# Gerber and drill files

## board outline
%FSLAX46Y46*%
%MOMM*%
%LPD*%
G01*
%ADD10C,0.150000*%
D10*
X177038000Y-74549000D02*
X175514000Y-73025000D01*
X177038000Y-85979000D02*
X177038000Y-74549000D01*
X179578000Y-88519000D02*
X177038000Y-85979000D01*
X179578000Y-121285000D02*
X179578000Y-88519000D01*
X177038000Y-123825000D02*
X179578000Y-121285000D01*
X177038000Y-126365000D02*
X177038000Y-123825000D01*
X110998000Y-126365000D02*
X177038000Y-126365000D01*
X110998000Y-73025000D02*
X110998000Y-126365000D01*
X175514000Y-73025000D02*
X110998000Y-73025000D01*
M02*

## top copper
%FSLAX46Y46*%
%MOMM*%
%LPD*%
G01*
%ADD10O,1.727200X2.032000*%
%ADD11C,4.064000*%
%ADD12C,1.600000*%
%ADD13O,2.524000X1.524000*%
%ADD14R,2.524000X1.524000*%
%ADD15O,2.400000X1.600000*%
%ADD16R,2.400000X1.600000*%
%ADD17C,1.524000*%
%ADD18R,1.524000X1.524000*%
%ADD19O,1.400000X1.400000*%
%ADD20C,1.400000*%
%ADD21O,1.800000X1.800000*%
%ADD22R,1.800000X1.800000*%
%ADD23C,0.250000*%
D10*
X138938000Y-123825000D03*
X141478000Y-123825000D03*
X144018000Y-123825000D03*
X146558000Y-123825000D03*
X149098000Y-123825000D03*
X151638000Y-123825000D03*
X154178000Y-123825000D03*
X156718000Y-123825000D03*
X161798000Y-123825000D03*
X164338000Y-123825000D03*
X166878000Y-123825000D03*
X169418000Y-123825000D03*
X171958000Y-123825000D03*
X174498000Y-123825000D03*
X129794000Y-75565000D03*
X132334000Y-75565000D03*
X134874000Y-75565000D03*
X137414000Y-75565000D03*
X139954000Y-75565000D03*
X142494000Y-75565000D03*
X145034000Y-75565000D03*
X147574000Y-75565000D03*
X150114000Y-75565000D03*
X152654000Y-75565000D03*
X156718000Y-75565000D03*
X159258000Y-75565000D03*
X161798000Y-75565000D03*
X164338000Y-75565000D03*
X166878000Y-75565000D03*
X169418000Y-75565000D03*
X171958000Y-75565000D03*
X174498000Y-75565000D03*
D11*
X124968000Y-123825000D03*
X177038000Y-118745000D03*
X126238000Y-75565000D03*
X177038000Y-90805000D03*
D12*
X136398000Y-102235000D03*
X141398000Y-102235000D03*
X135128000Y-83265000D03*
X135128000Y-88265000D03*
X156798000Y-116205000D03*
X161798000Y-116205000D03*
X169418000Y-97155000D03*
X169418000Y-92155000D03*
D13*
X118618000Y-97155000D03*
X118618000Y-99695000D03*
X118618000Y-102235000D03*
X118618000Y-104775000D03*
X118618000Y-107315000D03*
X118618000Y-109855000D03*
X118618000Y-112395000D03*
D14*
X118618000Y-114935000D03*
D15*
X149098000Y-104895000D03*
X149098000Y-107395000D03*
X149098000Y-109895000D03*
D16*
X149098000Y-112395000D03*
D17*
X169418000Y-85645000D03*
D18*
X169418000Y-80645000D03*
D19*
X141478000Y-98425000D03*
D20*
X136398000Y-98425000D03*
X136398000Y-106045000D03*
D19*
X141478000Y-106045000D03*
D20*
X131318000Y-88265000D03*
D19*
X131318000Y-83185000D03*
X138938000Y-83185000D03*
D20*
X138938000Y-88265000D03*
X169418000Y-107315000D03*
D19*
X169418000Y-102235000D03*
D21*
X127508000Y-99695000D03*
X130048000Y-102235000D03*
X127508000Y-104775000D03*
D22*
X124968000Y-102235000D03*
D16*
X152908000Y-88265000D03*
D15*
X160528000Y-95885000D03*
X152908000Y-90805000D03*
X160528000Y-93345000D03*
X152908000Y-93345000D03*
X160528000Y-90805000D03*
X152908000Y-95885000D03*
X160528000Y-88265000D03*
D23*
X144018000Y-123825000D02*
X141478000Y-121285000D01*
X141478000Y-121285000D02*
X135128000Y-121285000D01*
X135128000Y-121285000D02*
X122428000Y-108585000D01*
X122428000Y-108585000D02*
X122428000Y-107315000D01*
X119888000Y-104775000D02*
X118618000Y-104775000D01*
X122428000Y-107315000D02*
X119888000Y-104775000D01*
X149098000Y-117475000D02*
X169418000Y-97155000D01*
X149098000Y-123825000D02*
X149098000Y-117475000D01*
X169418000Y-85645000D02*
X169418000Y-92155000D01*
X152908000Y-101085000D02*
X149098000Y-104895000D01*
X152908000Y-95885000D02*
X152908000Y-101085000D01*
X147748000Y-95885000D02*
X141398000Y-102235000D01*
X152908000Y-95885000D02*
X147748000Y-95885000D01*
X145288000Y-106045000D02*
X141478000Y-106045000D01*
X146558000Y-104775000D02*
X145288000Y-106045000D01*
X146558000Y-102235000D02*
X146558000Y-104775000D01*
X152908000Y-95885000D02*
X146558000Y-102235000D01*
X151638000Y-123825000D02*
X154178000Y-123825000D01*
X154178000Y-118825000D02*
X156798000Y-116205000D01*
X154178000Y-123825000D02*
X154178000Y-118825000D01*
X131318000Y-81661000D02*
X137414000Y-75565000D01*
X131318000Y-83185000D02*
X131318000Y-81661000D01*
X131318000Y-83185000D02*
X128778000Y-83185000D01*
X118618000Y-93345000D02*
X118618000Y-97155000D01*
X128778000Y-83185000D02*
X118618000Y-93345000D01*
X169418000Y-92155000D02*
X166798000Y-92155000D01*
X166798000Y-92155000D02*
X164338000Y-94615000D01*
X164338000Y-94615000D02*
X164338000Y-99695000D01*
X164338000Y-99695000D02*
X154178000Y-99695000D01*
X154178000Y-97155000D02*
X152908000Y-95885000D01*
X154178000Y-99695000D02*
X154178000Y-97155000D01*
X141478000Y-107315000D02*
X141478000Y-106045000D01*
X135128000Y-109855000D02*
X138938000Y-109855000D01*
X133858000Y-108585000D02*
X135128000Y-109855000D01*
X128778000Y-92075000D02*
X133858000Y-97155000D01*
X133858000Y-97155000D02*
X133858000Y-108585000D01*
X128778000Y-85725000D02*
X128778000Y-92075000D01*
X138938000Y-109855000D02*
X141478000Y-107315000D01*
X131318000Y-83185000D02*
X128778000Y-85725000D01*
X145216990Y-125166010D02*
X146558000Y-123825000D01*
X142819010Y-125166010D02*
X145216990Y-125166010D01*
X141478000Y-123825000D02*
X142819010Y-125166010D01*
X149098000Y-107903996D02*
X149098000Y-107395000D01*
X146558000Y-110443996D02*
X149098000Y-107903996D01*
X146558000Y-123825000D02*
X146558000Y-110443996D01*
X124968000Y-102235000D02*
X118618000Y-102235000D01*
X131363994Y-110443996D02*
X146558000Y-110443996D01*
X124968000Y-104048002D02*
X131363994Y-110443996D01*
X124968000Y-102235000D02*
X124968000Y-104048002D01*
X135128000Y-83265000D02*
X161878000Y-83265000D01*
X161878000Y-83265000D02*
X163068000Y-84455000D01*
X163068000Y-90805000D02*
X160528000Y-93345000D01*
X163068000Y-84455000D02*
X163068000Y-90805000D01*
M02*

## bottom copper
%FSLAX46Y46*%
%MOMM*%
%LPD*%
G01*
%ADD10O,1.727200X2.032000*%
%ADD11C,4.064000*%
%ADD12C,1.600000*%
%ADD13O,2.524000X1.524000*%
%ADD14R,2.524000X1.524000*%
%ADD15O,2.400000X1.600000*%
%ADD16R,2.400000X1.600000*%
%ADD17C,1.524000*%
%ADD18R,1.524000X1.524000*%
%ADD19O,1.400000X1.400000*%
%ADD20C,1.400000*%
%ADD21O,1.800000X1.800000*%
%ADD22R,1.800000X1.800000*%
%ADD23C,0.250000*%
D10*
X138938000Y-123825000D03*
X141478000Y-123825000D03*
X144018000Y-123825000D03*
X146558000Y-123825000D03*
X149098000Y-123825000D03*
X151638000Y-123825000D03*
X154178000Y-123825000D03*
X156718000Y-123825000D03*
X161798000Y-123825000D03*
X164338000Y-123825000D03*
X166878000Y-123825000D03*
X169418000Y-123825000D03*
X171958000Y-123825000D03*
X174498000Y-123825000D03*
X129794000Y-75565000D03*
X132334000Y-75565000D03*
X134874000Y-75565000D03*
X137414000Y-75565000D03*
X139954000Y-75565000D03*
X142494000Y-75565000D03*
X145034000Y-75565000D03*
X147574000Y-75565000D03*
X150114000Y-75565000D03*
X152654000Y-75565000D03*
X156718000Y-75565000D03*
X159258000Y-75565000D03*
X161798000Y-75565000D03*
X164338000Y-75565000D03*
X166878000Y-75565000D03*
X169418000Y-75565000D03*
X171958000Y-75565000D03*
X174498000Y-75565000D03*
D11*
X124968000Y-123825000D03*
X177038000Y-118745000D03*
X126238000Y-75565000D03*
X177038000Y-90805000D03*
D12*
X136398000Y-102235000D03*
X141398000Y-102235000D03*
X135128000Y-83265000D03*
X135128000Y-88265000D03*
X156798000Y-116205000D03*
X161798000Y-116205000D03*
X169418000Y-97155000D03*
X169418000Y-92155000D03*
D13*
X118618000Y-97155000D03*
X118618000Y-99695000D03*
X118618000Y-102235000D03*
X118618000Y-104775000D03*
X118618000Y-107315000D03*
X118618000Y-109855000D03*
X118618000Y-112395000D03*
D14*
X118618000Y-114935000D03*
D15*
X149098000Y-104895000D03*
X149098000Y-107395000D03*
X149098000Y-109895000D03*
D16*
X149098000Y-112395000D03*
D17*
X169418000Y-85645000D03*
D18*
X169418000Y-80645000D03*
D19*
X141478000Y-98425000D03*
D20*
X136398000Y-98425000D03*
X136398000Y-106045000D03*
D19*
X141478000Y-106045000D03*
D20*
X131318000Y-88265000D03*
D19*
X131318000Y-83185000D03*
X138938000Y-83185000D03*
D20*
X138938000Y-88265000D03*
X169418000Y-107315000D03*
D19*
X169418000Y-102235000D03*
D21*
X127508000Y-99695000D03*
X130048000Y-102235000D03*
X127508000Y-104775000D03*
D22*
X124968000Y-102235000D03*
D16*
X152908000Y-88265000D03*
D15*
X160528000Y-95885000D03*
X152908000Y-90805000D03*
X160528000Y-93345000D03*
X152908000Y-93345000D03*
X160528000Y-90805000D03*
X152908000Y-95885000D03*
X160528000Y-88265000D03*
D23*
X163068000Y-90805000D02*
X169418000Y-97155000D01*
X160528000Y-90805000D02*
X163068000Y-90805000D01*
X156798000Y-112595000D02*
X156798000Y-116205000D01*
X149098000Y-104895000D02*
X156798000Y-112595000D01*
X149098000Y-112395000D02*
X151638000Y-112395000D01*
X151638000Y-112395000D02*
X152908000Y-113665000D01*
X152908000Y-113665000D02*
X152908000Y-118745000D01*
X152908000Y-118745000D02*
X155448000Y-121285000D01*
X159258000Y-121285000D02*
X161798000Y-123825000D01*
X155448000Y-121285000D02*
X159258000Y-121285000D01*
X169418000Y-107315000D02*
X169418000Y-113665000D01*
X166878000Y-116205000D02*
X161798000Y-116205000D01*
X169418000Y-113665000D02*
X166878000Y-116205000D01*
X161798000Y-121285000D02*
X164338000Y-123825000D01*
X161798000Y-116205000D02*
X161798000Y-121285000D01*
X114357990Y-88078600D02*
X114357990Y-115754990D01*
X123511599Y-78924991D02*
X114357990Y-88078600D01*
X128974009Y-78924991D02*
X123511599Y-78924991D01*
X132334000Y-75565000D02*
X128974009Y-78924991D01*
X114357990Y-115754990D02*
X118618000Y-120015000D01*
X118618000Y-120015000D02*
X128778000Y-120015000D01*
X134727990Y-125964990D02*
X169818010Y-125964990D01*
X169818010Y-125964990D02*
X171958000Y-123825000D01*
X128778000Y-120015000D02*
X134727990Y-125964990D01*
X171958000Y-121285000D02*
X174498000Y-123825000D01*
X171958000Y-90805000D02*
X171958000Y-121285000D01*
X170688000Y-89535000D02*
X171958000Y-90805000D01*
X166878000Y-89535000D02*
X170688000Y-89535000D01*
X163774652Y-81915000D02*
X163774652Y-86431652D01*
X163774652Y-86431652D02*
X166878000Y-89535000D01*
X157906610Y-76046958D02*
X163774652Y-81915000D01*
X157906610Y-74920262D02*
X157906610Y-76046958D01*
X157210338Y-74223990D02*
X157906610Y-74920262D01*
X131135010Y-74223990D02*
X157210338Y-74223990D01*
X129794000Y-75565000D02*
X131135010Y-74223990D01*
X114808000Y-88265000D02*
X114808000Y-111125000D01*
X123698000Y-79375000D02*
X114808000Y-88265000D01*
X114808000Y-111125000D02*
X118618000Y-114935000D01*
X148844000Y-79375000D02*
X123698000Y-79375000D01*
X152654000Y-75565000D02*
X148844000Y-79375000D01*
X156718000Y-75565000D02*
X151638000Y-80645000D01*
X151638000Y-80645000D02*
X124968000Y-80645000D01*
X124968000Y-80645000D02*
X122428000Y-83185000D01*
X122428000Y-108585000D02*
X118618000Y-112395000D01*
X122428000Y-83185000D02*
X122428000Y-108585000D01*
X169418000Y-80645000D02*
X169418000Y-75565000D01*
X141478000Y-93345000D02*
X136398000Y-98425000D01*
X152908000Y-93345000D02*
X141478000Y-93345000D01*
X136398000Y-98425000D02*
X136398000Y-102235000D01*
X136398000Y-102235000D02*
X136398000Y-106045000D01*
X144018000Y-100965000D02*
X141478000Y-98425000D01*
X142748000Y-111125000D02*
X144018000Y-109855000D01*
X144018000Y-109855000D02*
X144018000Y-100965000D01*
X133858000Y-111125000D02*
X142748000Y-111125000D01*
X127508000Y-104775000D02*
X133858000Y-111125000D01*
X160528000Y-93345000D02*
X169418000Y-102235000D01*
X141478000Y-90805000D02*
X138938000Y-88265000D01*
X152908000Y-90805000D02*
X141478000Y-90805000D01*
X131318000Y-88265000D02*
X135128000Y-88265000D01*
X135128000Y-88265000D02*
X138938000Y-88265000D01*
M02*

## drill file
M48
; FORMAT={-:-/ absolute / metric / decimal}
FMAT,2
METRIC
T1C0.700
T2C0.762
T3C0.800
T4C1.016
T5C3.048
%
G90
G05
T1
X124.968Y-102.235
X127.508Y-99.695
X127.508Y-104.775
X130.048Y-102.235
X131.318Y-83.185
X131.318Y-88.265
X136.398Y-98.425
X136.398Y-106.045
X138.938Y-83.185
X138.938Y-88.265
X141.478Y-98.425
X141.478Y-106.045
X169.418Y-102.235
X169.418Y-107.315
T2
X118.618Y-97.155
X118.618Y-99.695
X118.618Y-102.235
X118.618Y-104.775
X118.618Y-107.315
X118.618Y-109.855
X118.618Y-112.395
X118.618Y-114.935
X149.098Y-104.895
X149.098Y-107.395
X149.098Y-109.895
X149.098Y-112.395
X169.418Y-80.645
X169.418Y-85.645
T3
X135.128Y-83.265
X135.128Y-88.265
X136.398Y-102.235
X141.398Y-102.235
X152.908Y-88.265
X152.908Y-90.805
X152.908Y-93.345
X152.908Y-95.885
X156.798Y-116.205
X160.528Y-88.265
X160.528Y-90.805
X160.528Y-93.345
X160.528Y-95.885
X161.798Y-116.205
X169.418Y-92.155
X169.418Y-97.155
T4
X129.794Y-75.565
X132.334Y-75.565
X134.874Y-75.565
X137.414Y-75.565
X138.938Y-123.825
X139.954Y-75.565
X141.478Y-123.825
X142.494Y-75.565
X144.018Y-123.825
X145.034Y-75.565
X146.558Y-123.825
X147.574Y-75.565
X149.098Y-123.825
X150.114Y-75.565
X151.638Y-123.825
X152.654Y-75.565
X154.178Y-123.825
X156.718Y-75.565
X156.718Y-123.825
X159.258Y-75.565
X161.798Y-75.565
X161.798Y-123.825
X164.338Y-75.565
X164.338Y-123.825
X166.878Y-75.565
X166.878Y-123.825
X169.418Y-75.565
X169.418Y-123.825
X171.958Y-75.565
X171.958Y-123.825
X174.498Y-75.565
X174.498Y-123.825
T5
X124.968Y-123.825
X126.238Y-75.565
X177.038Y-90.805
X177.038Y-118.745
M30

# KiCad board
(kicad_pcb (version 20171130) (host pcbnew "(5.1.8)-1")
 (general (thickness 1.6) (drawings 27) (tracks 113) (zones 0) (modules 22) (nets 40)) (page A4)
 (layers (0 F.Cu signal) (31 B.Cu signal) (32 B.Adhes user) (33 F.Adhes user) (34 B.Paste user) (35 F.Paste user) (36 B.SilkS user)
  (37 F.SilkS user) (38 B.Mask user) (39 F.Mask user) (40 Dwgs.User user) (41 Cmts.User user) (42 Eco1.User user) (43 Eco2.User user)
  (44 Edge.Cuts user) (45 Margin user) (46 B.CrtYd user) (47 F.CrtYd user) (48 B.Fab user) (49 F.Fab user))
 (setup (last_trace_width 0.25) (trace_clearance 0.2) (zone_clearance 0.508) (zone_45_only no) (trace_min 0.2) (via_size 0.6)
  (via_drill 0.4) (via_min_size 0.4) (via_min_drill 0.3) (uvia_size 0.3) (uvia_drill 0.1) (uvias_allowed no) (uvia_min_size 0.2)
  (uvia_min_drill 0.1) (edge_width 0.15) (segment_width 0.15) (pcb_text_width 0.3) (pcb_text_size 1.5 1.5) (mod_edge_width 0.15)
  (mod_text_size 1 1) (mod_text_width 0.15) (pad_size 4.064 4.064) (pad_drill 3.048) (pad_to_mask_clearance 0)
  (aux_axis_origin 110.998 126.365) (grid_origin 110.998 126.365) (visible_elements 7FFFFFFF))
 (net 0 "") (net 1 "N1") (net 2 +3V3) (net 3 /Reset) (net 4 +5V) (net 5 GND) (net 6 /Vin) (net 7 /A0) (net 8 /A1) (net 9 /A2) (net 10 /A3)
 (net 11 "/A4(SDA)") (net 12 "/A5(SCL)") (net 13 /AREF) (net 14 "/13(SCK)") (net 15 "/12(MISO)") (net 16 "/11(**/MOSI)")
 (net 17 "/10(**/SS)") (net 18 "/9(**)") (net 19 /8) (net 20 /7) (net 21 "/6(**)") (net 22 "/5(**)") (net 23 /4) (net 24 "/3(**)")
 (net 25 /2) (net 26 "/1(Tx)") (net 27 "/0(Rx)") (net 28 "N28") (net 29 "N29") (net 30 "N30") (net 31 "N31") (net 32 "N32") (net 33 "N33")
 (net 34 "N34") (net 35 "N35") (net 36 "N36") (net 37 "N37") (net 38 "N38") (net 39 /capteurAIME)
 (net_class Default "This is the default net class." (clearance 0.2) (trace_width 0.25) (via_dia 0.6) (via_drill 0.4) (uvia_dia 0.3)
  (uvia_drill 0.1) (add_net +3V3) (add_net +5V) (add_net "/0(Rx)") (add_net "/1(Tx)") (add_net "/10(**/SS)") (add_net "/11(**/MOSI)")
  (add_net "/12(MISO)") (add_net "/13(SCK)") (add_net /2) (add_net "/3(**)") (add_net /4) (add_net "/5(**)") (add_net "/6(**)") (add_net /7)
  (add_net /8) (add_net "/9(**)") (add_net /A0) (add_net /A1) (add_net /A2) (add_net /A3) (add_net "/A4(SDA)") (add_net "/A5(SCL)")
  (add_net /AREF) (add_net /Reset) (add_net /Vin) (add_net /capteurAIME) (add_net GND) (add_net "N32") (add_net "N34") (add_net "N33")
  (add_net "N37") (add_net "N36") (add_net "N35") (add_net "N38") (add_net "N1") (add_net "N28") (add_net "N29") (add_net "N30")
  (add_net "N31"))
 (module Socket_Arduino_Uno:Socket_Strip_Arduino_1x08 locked (layer F.Cu) (at 138.938 123.825)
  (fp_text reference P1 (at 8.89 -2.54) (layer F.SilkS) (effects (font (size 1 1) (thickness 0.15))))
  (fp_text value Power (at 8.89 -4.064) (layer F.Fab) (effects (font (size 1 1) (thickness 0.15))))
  (pad 1 thru_hole oval (at 0 0) (size 1.7272 2.032) (drill 1.016) (layers *.Cu *.Mask F.SilkS) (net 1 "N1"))
  (pad 2 thru_hole oval (at 2.54 0) (size 1.7272 2.032) (drill 1.016) (layers *.Cu *.Mask F.SilkS) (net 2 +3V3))
  (pad 3 thru_hole oval (at 5.08 0) (size 1.7272 2.032) (drill 1.016) (layers *.Cu *.Mask F.SilkS) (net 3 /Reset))
  (pad 4 thru_hole oval (at 7.62 0) (size 1.7272 2.032) (drill 1.016) (layers *.Cu *.Mask F.SilkS) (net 2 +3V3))
  (pad 5 thru_hole oval (at 10.16 0) (size 1.7272 2.032) (drill 1.016) (layers *.Cu *.Mask F.SilkS) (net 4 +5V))
  (pad 6 thru_hole oval (at 12.7 0) (size 1.7272 2.032) (drill 1.016) (layers *.Cu *.Mask F.SilkS) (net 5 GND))
  (pad 7 thru_hole oval (at 15.24 0) (size 1.7272 2.032) (drill 1.016) (layers *.Cu *.Mask F.SilkS) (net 5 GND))
  (pad 8 thru_hole oval (at 17.78 0) (size 1.7272 2.032) (drill 1.016) (layers *.Cu *.Mask F.SilkS) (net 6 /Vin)))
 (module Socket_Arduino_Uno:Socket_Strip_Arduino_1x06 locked (layer F.Cu) (at 161.798 123.825)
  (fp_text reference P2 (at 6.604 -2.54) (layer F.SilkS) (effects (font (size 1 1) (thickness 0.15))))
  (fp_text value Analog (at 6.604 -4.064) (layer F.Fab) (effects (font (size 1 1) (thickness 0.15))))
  (pad 1 thru_hole oval (at 0 0) (size 1.7272 2.032) (drill 1.016) (layers *.Cu *.Mask F.SilkS) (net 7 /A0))
  (pad 2 thru_hole oval (at 2.54 0) (size 1.7272 2.032) (drill 1.016) (layers *.Cu *.Mask F.SilkS) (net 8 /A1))
  (pad 3 thru_hole oval (at 5.08 0) (size 1.7272 2.032) (drill 1.016) (layers *.Cu *.Mask F.SilkS) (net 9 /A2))
  (pad 4 thru_hole oval (at 7.62 0) (size 1.7272 2.032) (drill 1.016) (layers *.Cu *.Mask F.SilkS) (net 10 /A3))
  (pad 5 thru_hole oval (at 10.16 0) (size 1.7272 2.032) (drill 1.016) (layers *.Cu *.Mask F.SilkS) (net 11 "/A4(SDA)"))
  (pad 6 thru_hole oval (at 12.7 0) (size 1.7272 2.032) (drill 1.016) (layers *.Cu *.Mask F.SilkS) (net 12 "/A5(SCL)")))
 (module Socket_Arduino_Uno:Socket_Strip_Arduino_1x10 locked (layer F.Cu) (at 129.794 75.565)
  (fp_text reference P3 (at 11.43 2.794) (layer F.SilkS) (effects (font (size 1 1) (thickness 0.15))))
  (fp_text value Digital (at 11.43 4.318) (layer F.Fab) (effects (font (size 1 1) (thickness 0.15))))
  (pad 1 thru_hole oval (at 0 0) (size 1.7272 2.032) (drill 1.016) (layers *.Cu *.Mask F.SilkS) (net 12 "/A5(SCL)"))
  (pad 2 thru_hole oval (at 2.54 0) (size 1.7272 2.032) (drill 1.016) (layers *.Cu *.Mask F.SilkS) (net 11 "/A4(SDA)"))
  (pad 3 thru_hole oval (at 5.08 0) (size 1.7272 2.032) (drill 1.016) (layers *.Cu *.Mask F.SilkS) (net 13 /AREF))
  (pad 4 thru_hole oval (at 7.62 0) (size 1.7272 2.032) (drill 1.016) (layers *.Cu *.Mask F.SilkS) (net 5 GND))
  (pad 5 thru_hole oval (at 10.16 0) (size 1.7272 2.032) (drill 1.016) (layers *.Cu *.Mask F.SilkS) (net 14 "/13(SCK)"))
  (pad 6 thru_hole oval (at 12.7 0) (size 1.7272 2.032) (drill 1.016) (layers *.Cu *.Mask F.SilkS) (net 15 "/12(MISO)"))
  (pad 7 thru_hole oval (at 15.24 0) (size 1.7272 2.032) (drill 1.016) (layers *.Cu *.Mask F.SilkS) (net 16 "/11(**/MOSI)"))
  (pad 8 thru_hole oval (at 17.78 0) (size 1.7272 2.032) (drill 1.016) (layers *.Cu *.Mask F.SilkS) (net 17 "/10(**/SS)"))
  (pad 9 thru_hole oval (at 20.32 0) (size 1.7272 2.032) (drill 1.016) (layers *.Cu *.Mask F.SilkS) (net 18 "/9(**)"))
  (pad 10 thru_hole oval (at 22.86 0) (size 1.7272 2.032) (drill 1.016) (layers *.Cu *.Mask F.SilkS) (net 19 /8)))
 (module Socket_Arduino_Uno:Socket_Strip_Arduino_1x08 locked (layer F.Cu) (at 156.718 75.565)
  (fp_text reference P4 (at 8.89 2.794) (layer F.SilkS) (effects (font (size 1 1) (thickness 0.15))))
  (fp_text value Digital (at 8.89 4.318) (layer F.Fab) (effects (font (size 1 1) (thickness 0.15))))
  (pad 1 thru_hole oval (at 0 0) (size 1.7272 2.032) (drill 1.016) (layers *.Cu *.Mask F.SilkS) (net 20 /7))
  (pad 2 thru_hole oval (at 2.54 0) (size 1.7272 2.032) (drill 1.016) (layers *.Cu *.Mask F.SilkS) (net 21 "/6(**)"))
  (pad 3 thru_hole oval (at 5.08 0) (size 1.7272 2.032) (drill 1.016) (layers *.Cu *.Mask F.SilkS) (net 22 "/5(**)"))
  (pad 4 thru_hole oval (at 7.62 0) (size 1.7272 2.032) (drill 1.016) (layers *.Cu *.Mask F.SilkS) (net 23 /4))
  (pad 5 thru_hole oval (at 10.16 0) (size 1.7272 2.032) (drill 1.016) (layers *.Cu *.Mask F.SilkS) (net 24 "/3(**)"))
  (pad 6 thru_hole oval (at 12.7 0) (size 1.7272 2.032) (drill 1.016) (layers *.Cu *.Mask F.SilkS) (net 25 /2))
  (pad 7 thru_hole oval (at 15.24 0) (size 1.7272 2.032) (drill 1.016) (layers *.Cu *.Mask F.SilkS) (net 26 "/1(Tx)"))
  (pad 8 thru_hole oval (at 17.78 0) (size 1.7272 2.032) (drill 1.016) (layers *.Cu *.Mask F.SilkS) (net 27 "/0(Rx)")))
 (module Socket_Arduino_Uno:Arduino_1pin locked (layer F.Cu) (at 124.968 123.825)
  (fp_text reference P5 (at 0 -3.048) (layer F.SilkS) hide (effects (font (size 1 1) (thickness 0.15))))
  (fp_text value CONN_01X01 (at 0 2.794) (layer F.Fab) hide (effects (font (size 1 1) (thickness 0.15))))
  (pad 1 thru_hole circle (at 0 0) (size 4.064 4.064) (drill 3.048) (layers *.Cu *.Mask F.SilkS) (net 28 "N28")))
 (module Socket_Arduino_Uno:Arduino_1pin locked (layer F.Cu) (at 177.038 118.745)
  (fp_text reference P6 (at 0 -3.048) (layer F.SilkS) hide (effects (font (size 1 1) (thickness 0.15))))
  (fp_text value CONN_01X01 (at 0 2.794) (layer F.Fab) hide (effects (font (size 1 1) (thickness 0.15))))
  (pad 1 thru_hole circle (at 0 0) (size 4.064 4.064) (drill 3.048) (layers *.Cu *.Mask F.SilkS) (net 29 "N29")))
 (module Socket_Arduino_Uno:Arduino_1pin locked (layer F.Cu) (at 126.238 75.565)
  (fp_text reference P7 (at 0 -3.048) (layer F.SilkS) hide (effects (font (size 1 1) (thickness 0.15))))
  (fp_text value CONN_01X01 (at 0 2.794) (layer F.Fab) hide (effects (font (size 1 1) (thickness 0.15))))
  (pad 1 thru_hole circle (at 0 0) (size 4.064 4.064) (drill 3.048) (layers *.Cu *.Mask F.SilkS) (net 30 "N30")))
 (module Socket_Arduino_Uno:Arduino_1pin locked (layer F.Cu) (at 177.038 90.805)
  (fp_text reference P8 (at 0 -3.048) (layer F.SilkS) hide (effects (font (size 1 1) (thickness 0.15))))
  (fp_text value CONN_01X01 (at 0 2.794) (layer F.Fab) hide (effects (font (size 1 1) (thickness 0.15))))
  (pad 1 thru_hole circle (at 0 0) (size 4.064 4.064) (drill 3.048) (layers *.Cu *.Mask F.SilkS) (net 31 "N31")))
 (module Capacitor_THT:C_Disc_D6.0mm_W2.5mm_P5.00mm (layer F.Cu) (at 136.398 102.235)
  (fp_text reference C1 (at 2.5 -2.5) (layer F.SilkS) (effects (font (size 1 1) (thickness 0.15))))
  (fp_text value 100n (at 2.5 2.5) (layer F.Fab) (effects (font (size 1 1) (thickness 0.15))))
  (pad 1 thru_hole circle (at 0 0) (size 1.6 1.6) (drill 0.8) (layers *.Cu *.Mask) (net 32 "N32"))
  (pad 2 thru_hole circle (at 5 0) (size 1.6 1.6) (drill 0.8) (layers *.Cu *.Mask) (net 5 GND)))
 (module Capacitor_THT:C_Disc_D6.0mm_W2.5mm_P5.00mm (layer F.Cu) (at 135.128 88.265 90)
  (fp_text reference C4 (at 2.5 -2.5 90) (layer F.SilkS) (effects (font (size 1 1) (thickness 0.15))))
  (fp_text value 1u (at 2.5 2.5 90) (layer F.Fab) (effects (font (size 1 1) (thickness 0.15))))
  (pad 2 thru_hole circle (at 5 0 90) (size 1.6 1.6) (drill 0.8) (layers *.Cu *.Mask) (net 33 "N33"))
  (pad 1 thru_hole circle (at 0 0 90) (size 1.6 1.6) (drill 0.8) (layers *.Cu *.Mask) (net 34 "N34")))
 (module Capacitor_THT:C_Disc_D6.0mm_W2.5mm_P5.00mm (layer F.Cu) (at 161.798 116.205 180)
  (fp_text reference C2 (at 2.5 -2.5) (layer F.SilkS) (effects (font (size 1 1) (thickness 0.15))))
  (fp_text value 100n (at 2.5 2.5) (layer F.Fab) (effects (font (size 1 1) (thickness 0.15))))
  (pad 2 thru_hole circle (at 5 0 180) (size 1.6 1.6) (drill 0.8) (layers *.Cu *.Mask) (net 5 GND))
  (pad 1 thru_hole circle (at 0 0 180) (size 1.6 1.6) (drill 0.8) (layers *.Cu *.Mask) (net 8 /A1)))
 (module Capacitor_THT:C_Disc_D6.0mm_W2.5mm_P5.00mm (layer F.Cu) (at 169.418 97.155 90)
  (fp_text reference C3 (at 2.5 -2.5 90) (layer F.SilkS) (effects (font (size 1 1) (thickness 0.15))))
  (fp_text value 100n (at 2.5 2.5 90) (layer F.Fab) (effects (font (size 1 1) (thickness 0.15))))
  (pad 1 thru_hole circle (at 0 0 90) (size 1.6 1.6) (drill 0.8) (layers *.Cu *.Mask) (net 4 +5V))
  (pad 2 thru_hole circle (at 5 0 90) (size 1.6 1.6) (drill 0.8) (layers *.Cu *.Mask) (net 5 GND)))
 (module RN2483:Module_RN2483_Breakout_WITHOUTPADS (layer F.Cu) (at 118.618 114.935 90)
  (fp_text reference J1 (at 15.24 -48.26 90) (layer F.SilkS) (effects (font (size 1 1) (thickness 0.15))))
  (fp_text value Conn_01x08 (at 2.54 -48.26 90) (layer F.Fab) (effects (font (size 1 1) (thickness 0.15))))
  (pad 8 thru_hole oval (at 17.78 0 90) (size 1.524 2.524) (drill 0.762) (layers *.Cu *.Mask) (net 5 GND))
  (pad 7 thru_hole oval (at 15.24 0 90) (size 1.524 2.524) (drill 0.762) (layers *.Cu *.Mask) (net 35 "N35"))
  (pad 6 thru_hole oval (at 12.7 0 90) (size 1.524 2.524) (drill 0.762) (layers *.Cu *.Mask) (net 2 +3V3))
  (pad 5 thru_hole oval (at 10.16 0 90) (size 1.524 2.524) (drill 0.762) (layers *.Cu *.Mask) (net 3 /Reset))
  (pad 4 thru_hole oval (at 7.62 0 90) (size 1.524 2.524) (drill 0.762) (layers *.Cu *.Mask) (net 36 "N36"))
  (pad 3 thru_hole oval (at 5.08 0 90) (size 1.524 2.524) (drill 0.762) (layers *.Cu *.Mask) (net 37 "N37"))
  (pad 2 thru_hole oval (at 2.54 0 90) (size 1.524 2.524) (drill 0.762) (layers *.Cu *.Mask) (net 20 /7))
  (pad 1 thru_hole rect (at 0 0 90) (size 1.524 2.524) (drill 0.762) (layers *.Cu *.Mask) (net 19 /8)))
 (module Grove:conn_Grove (layer F.Cu) (at 149.098 112.395 90)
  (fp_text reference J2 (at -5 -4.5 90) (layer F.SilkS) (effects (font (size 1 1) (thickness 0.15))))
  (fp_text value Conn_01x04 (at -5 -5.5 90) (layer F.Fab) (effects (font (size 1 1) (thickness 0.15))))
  (pad 4 thru_hole oval (at 7.5 0 90) (size 1.6 2.4) (drill 0.762) (layers *.Cu *.Mask) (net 5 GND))
  (pad 3 thru_hole oval (at 5 0 90) (size 1.6 2.4) (drill 0.762) (layers *.Cu *.Mask) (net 2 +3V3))
  (pad 2 thru_hole oval (at 2.5 0 90) (size 1.6 2.4) (drill 0.762) (layers *.Cu *.Mask) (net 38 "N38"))
  (pad 1 thru_hole rect (at 0 0 90) (size 1.6 2.4) (drill 0.762) (layers *.Cu *.Mask) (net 7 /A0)))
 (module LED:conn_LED (layer F.Cu) (at 169.418 80.645 270)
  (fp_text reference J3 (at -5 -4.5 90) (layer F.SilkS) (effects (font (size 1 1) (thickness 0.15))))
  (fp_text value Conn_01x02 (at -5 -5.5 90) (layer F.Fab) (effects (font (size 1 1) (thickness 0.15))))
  (pad 2 thru_hole circle (at 5 0 270) (size 1.524 1.524) (drill 0.762) (layers *.Cu *.Mask) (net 5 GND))
  (pad 1 thru_hole rect (at 0 0 270) (size 1.524 1.524) (drill 0.762) (layers *.Cu *.Mask) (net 25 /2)))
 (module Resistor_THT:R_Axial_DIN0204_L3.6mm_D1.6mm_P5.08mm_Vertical (layer F.Cu) (at 136.398 98.425)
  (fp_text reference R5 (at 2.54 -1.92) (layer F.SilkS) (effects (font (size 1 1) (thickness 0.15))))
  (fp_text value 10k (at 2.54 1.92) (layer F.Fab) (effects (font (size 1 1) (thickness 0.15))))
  (pad 2 thru_hole oval (at 5.08 0) (size 1.4 1.4) (drill 0.7) (layers *.Cu *.Mask) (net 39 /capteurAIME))
  (pad 1 thru_hole circle (at 0 0) (size 1.4 1.4) (drill 0.7) (layers *.Cu *.Mask) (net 32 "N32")))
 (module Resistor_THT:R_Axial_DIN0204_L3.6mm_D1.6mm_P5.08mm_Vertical (layer F.Cu) (at 136.398 106.045)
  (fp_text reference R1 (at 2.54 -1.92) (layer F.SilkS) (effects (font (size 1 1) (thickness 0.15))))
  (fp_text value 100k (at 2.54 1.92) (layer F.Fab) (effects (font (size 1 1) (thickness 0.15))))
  (pad 1 thru_hole circle (at 0 0) (size 1.4 1.4) (drill 0.7) (layers *.Cu *.Mask) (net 32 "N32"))
  (pad 2 thru_hole oval (at 5.08 0) (size 1.4 1.4) (drill 0.7) (layers *.Cu *.Mask) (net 5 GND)))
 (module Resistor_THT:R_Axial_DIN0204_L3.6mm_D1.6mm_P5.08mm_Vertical (layer F.Cu) (at 131.318 88.265 90)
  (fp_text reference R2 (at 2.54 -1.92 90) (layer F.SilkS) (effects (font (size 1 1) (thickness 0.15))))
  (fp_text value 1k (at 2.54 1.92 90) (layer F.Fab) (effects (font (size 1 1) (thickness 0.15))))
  (pad 1 thru_hole circle (at 0 0 90) (size 1.4 1.4) (drill 0.7) (layers *.Cu *.Mask) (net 34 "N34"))
  (pad 2 thru_hole oval (at 5.08 0 90) (size 1.4 1.4) (drill 0.7) (layers *.Cu *.Mask) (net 5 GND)))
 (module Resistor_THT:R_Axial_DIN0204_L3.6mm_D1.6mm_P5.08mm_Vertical (layer F.Cu) (at 138.938 88.265 90)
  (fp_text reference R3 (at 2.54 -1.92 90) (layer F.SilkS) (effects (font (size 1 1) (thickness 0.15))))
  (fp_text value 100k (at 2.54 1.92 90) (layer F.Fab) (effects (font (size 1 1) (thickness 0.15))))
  (pad 2 thru_hole oval (at 5.08 0 90) (size 1.4 1.4) (drill 0.7) (layers *.Cu *.Mask) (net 33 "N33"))
  (pad 1 thru_hole circle (at 0 0 90) (size 1.4 1.4) (drill 0.7) (layers *.Cu *.Mask) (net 34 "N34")))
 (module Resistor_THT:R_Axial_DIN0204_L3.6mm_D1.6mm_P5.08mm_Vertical (layer F.Cu) (at 169.418 107.315 90)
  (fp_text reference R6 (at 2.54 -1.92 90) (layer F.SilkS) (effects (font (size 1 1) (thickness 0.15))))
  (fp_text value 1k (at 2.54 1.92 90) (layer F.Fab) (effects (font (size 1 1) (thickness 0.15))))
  (pad 1 thru_hole circle (at 0 0 90) (size 1.4 1.4) (drill 0.7) (layers *.Cu *.Mask) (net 8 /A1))
  (pad 2 thru_hole oval (at 5.08 0 90) (size 1.4 1.4) (drill 0.7) (layers *.Cu *.Mask) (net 33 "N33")))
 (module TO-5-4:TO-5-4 (layer F.Cu) (at 124.968 102.235)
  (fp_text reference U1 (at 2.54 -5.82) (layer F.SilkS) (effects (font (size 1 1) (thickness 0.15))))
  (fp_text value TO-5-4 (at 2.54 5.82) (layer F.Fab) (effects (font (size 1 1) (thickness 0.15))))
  (pad 4 thru_hole oval (at 2.54 -2.54) (size 1.8 1.8) (drill 0.7) (layers *.Cu *.Mask))
  (pad 3 thru_hole oval (at 5.08 0) (size 1.8 1.8) (drill 0.7) (layers *.Cu *.Mask))
  (pad 2 thru_hole oval (at 2.54 2.54) (size 1.8 1.8) (drill 0.7) (layers *.Cu *.Mask) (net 39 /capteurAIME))
  (pad 1 thru_hole rect (at 0 0) (size 1.8 1.8) (drill 0.7) (layers *.Cu *.Mask) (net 2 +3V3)))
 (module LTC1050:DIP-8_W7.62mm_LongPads (layer F.Cu) (at 152.908 88.265)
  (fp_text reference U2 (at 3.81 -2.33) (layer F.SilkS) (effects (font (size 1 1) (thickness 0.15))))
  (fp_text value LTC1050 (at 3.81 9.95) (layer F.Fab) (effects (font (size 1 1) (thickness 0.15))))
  (pad 1 thru_hole rect (at 0 0) (size 2.4 1.6) (drill 0.8) (layers *.Cu *.Mask))
  (pad 5 thru_hole oval (at 7.62 7.62) (size 2.4 1.6) (drill 0.8) (layers *.Cu *.Mask))
  (pad 2 thru_hole oval (at 0 2.54) (size 2.4 1.6) (drill 0.8) (layers *.Cu *.Mask) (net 34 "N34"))
  (pad 6 thru_hole oval (at 7.62 5.08) (size 2.4 1.6) (drill 0.8) (layers *.Cu *.Mask) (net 33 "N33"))
  (pad 3 thru_hole oval (at 0 5.08) (size 2.4 1.6) (drill 0.8) (layers *.Cu *.Mask) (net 32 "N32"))
  (pad 7 thru_hole oval (at 7.62 2.54) (size 2.4 1.6) (drill 0.8) (layers *.Cu *.Mask) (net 4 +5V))
  (pad 4 thru_hole oval (at 0 7.62) (size 2.4 1.6) (drill 0.8) (layers *.Cu *.Mask) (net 5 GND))
  (pad 8 thru_hole oval (at 7.62 0) (size 2.4 1.6) (drill 0.8) (layers *.Cu *.Mask)))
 (gr_line (start 177.038 74.549) (end 175.514 73.025) (angle 90) (layer Edge.Cuts) (width 0.15))
 (gr_line (start 177.038 85.979) (end 177.038 74.549) (angle 90) (layer Edge.Cuts) (width 0.15))
 (gr_line (start 179.578 88.519) (end 177.038 85.979) (angle 90) (layer Edge.Cuts) (width 0.15))
 (gr_line (start 179.578 121.285) (end 179.578 88.519) (angle 90) (layer Edge.Cuts) (width 0.15))
 (gr_line (start 177.038 123.825) (end 179.578 121.285) (angle 90) (layer Edge.Cuts) (width 0.15))
 (gr_line (start 177.038 126.365) (end 177.038 123.825) (angle 90) (layer Edge.Cuts) (width 0.15))
 (gr_line (start 110.998 126.365) (end 177.038 126.365) (angle 90) (layer Edge.Cuts) (width 0.15))
 (gr_line (start 110.998 73.025) (end 110.998 126.365) (angle 90) (layer Edge.Cuts) (width 0.15))
 (gr_line (start 175.514 73.025) (end 110.998 73.025) (angle 90) (layer Edge.Cuts) (width 0.15))
 (segment (start 144.018 123.825) (end 141.478 121.285) (width 0.25) (layer F.Cu) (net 3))
 (segment (start 141.478 121.285) (end 135.128 121.285) (width 0.25) (layer F.Cu) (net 3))
 (segment (start 135.128 121.285) (end 122.428 108.585) (width 0.25) (layer F.Cu) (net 3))
 (segment (start 122.428 108.585) (end 122.428 107.315) (width 0.25) (layer F.Cu) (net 3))
 (segment (start 119.888 104.775) (end 118.618 104.775) (width 0.25) (layer F.Cu) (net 3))
 (segment (start 122.428 107.315) (end 119.888 104.775) (width 0.25) (layer F.Cu) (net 3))
 (segment (start 149.098 117.475) (end 169.418 97.155) (width 0.25) (layer F.Cu) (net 4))
 (segment (start 149.098 123.825) (end 149.098 117.475) (width 0.25) (layer F.Cu) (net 4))
 (segment (start 163.068 90.805) (end 169.418 97.155) (width 0.25) (layer B.Cu) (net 4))
 (segment (start 160.528 90.805) (end 163.068 90.805) (width 0.25) (layer B.Cu) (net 4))
 (segment (start 169.418 85.645) (end 169.418 92.155) (width 0.25) (layer F.Cu) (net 5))
 (segment (start 152.908 101.085) (end 149.098 104.895) (width 0.25) (layer F.Cu) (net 5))
 (segment (start 152.908 95.885) (end 152.908 101.085) (width 0.25) (layer F.Cu) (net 5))
 (segment (start 147.748 95.885) (end 141.398 102.235) (width 0.25) (layer F.Cu) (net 5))
 (segment (start 152.908 95.885) (end 147.748 95.885) (width 0.25) (layer F.Cu) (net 5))
 (segment (start 145.288 106.045) (end 141.478 106.045) (width 0.25) (layer F.Cu) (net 5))
 (segment (start 146.558 104.775) (end 145.288 106.045) (width 0.25) (layer F.Cu) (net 5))
 (segment (start 146.558 102.235) (end 146.558 104.775) (width 0.25) (layer F.Cu) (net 5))
 (segment (start 152.908 95.885) (end 146.558 102.235) (width 0.25) (layer F.Cu) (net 5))
 (segment (start 151.638 123.825) (end 154.178 123.825) (width 0.25) (layer F.Cu) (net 5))
 (segment (start 154.178 118.825) (end 156.798 116.205) (width 0.25) (layer F.Cu) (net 5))
 (segment (start 154.178 123.825) (end 154.178 118.825) (width 0.25) (layer F.Cu) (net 5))
 (segment (start 131.318 81.661) (end 137.414 75.565) (width 0.25) (layer F.Cu) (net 5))
 (segment (start 131.318 83.185) (end 131.318 81.661) (width 0.25) (layer F.Cu) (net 5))
 (segment (start 131.318 83.185) (end 128.778 83.185) (width 0.25) (layer F.Cu) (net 5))
 (segment (start 118.618 93.345) (end 118.618 97.155) (width 0.25) (layer F.Cu) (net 5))
 (segment (start 128.778 83.185) (end 118.618 93.345) (width 0.25) (layer F.Cu) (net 5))
 (segment (start 169.418 92.155) (end 166.798 92.155) (width 0.25) (layer F.Cu) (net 5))
 (segment (start 166.798 92.155) (end 164.338 94.615) (width 0.25) (layer F.Cu) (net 5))
 (segment (start 164.338 94.615) (end 164.338 99.695) (width 0.25) (layer F.Cu) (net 5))
 (segment (start 164.338 99.695) (end 154.178 99.695) (width 0.25) (layer F.Cu) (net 5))
 (segment (start 154.178 97.155) (end 152.908 95.885) (width 0.25) (layer F.Cu) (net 5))
 (segment (start 154.178 99.695) (end 154.178 97.155) (width 0.25) (layer F.Cu) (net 5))
 (segment (start 141.478 107.315) (end 141.478 106.045) (width 0.25) (layer F.Cu) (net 5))
 (segment (start 135.128 109.855) (end 138.938 109.855) (width 0.25) (layer F.Cu) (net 5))
 (segment (start 133.858 108.585) (end 135.128 109.855) (width 0.25) (layer F.Cu) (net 5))
 (segment (start 128.778 92.075) (end 133.858 97.155) (width 0.25) (layer F.Cu) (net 5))
 (segment (start 133.858 97.155) (end 133.858 108.585) (width 0.25) (layer F.Cu) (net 5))
 (segment (start 128.778 85.725) (end 128.778 92.075) (width 0.25) (layer F.Cu) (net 5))
 (segment (start 138.938 109.855) (end 141.478 107.315) (width 0.25) (layer F.Cu) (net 5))
 (segment (start 131.318 83.185) (end 128.778 85.725) (width 0.25) (layer F.Cu) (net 5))
 (segment (start 156.798 112.595) (end 156.798 116.205) (width 0.25) (layer B.Cu) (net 5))
 (segment (start 149.098 104.895) (end 156.798 112.595) (width 0.25) (layer B.Cu) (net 5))
 (segment (start 149.098 112.395) (end 151.638 112.395) (width 0.25) (layer B.Cu) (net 7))
 (segment (start 151.638 112.395) (end 152.908 113.665) (width 0.25) (layer B.Cu) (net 7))
 (segment (start 152.908 113.665) (end 152.908 118.745) (width 0.25) (layer B.Cu) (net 7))
 (segment (start 152.908 118.745) (end 155.448 121.285) (width 0.25) (layer B.Cu) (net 7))
 (segment (start 159.258 121.285) (end 161.798 123.825) (width 0.25) (layer B.Cu) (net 7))
 (segment (start 155.448 121.285) (end 159.258 121.285) (width 0.25) (layer B.Cu) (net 7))
 (segment (start 169.418 107.315) (end 169.418 113.665) (width 0.25) (layer B.Cu) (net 8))
 (segment (start 166.878 116.205) (end 161.798 116.205) (width 0.25) (layer B.Cu) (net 8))
 (segment (start 169.418 113.665) (end 166.878 116.205) (width 0.25) (layer B.Cu) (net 8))
 (segment (start 161.798 121.285) (end 164.338 123.825) (width 0.25) (layer B.Cu) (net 8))
 (segment (start 161.798 116.205) (end 161.798 121.285) (width 0.25) (layer B.Cu) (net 8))
 (segment (start 114.35799 88.0786) (end 114.35799 115.75499) (width 0.25) (layer B.Cu) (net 11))
 (segment (start 123.511599 78.924991) (end 114.35799 88.0786) (width 0.25) (layer B.Cu) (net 11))
 (segment (start 128.974009 78.924991) (end 123.511599 78.924991) (width 0.25) (layer B.Cu) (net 11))
 (segment (start 132.334 75.565) (end 128.974009 78.924991) (width 0.25) (layer B.Cu) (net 11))
 (segment (start 114.35799 115.75499) (end 118.618 120.015) (width 0.25) (layer B.Cu) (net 11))
 (segment (start 118.618 120.015) (end 128.778 120.015) (width 0.25) (layer B.Cu) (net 11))
 (segment (start 134.72799 125.96499) (end 169.81801 125.96499) (width 0.25) (layer B.Cu) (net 11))
 (segment (start 169.81801 125.96499) (end 171.958 123.825) (width 0.25) (layer B.Cu) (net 11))
 (segment (start 128.778 120.015) (end 134.72799 125.96499) (width 0.25) (layer B.Cu) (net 11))
 (segment (start 171.958 121.285) (end 174.498 123.825) (width 0.25) (layer B.Cu) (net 12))
 (segment (start 171.958 90.805) (end 171.958 121.285) (width 0.25) (layer B.Cu) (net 12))
 (segment (start 170.688 89.535) (end 171.958 90.805) (width 0.25) (layer B.Cu) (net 12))
 (segment (start 166.878 89.535) (end 170.688 89.535) (width 0.25) (layer B.Cu) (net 12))
 (segment (start 163.774652 81.915) (end 163.774652 86.431652) (width 0.25) (layer B.Cu) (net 12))
 (segment (start 163.774652 86.431652) (end 166.878 89.535) (width 0.25) (layer B.Cu) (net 12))
 (segment (start 157.90661 76.046958) (end 163.774652 81.915) (width 0.25) (layer B.Cu) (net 12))
 (segment (start 157.90661 74.920262) (end 157.90661 76.046958) (width 0.25) (layer B.Cu) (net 12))
 (segment (start 157.210338 74.22399) (end 157.90661 74.920262) (width 0.25) (layer B.Cu) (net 12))
 (segment (start 131.13501 74.22399) (end 157.210338 74.22399) (width 0.25) (layer B.Cu) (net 12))
 (segment (start 129.794 75.565) (end 131.13501 74.22399) (width 0.25) (layer B.Cu) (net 12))
 (segment (start 114.808 88.265) (end 114.808 111.125) (width 0.25) (layer B.Cu) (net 19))
 (segment (start 123.698 79.375) (end 114.808 88.265) (width 0.25) (layer B.Cu) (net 19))
 (segment (start 114.808 111.125) (end 118.618 114.935) (width 0.25) (layer B.Cu) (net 19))
 (segment (start 148.844 79.375) (end 123.698 79.375) (width 0.25) (layer B.Cu) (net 19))
 (segment (start 152.654 75.565) (end 148.844 79.375) (width 0.25) (layer B.Cu) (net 19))
 (segment (start 156.718 75.565) (end 151.638 80.645) (width 0.25) (layer B.Cu) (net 20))
 (segment (start 151.638 80.645) (end 124.968 80.645) (width 0.25) (layer B.Cu) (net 20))
 (segment (start 124.968 80.645) (end 122.428 83.185) (width 0.25) (layer B.Cu) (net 20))
 (segment (start 122.428 108.585) (end 118.618 112.395) (width 0.25) (layer B.Cu) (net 20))
 (segment (start 122.428 83.185) (end 122.428 108.585) (width 0.25) (layer B.Cu) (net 20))
 (segment (start 169.418 80.645) (end 169.418 75.565) (width 0.25) (layer B.Cu) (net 25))
 (segment (start 145.21699 125.16601) (end 146.558 123.825) (width 0.25) (layer F.Cu) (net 2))
 (segment (start 142.81901 125.16601) (end 145.21699 125.16601) (width 0.25) (layer F.Cu) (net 2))
 (segment (start 141.478 123.825) (end 142.81901 125.16601) (width 0.25) (layer F.Cu) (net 2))
 (segment (start 149.098 107.903996) (end 149.098 107.395) (width 0.25) (layer F.Cu) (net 2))
 (segment (start 146.558 110.443996) (end 149.098 107.903996) (width 0.25) (layer F.Cu) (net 2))
 (segment (start 146.558 123.825) (end 146.558 110.443996) (width 0.25) (layer F.Cu) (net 2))
 (segment (start 124.968 102.235) (end 118.618 102.235) (width 0.25) (layer F.Cu) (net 2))
 (segment (start 131.363994 110.443996) (end 146.558 110.443996) (width 0.25) (layer F.Cu) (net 2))
 (segment (start 124.968 104.048002) (end 131.363994 110.443996) (width 0.25) (layer F.Cu) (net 2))
 (segment (start 124.968 102.235) (end 124.968 104.048002) (width 0.25) (layer F.Cu) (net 2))
 (segment (start 141.478 93.345) (end 136.398 98.425) (width 0.25) (layer B.Cu) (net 32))
 (segment (start 152.908 93.345) (end 141.478 93.345) (width 0.25) (layer B.Cu) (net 32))
 (segment (start 136.398 98.425) (end 136.398 102.235) (width 0.25) (layer B.Cu) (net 32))
 (segment (start 136.398 102.235) (end 136.398 106.045) (width 0.25) (layer B.Cu) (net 32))
 (segment (start 144.018 100.965) (end 141.478 98.425) (width 0.25) (layer B.Cu) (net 39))
 (segment (start 142.748 111.125) (end 144.018 109.855) (width 0.25) (layer B.Cu) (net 39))
 (segment (start 144.018 109.855) (end 144.018 100.965) (width 0.25) (layer B.Cu) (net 39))
 (segment (start 133.858 111.125) (end 142.748 111.125) (width 0.25) (layer B.Cu) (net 39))
 (segment (start 127.508 104.775) (end 133.858 111.125) (width 0.25) (layer B.Cu) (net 39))
 (segment (start 135.128 83.265) (end 161.878 83.265) (width 0.25) (layer F.Cu) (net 33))
 (segment (start 161.878 83.265) (end 163.068 84.455) (width 0.25) (layer F.Cu) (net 33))
 (segment (start 163.068 90.805) (end 160.528 93.345) (width 0.25) (layer F.Cu) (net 33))
 (segment (start 163.068 84.455) (end 163.068 90.805) (width 0.25) (layer F.Cu) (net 33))
 (segment (start 160.528 93.345) (end 169.418 102.235) (width 0.25) (layer B.Cu) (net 33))
 (segment (start 141.478 90.805) (end 138.938 88.265) (width 0.25) (layer B.Cu) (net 34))
 (segment (start 152.908 90.805) (end 141.478 90.805) (width 0.25) (layer B.Cu) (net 34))
 (segment (start 131.318 88.265) (end 135.128 88.265) (width 0.25) (layer B.Cu) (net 34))
 (segment (start 135.128 88.265) (end 138.938 88.265) (width 0.25) (layer B.Cu) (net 34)))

